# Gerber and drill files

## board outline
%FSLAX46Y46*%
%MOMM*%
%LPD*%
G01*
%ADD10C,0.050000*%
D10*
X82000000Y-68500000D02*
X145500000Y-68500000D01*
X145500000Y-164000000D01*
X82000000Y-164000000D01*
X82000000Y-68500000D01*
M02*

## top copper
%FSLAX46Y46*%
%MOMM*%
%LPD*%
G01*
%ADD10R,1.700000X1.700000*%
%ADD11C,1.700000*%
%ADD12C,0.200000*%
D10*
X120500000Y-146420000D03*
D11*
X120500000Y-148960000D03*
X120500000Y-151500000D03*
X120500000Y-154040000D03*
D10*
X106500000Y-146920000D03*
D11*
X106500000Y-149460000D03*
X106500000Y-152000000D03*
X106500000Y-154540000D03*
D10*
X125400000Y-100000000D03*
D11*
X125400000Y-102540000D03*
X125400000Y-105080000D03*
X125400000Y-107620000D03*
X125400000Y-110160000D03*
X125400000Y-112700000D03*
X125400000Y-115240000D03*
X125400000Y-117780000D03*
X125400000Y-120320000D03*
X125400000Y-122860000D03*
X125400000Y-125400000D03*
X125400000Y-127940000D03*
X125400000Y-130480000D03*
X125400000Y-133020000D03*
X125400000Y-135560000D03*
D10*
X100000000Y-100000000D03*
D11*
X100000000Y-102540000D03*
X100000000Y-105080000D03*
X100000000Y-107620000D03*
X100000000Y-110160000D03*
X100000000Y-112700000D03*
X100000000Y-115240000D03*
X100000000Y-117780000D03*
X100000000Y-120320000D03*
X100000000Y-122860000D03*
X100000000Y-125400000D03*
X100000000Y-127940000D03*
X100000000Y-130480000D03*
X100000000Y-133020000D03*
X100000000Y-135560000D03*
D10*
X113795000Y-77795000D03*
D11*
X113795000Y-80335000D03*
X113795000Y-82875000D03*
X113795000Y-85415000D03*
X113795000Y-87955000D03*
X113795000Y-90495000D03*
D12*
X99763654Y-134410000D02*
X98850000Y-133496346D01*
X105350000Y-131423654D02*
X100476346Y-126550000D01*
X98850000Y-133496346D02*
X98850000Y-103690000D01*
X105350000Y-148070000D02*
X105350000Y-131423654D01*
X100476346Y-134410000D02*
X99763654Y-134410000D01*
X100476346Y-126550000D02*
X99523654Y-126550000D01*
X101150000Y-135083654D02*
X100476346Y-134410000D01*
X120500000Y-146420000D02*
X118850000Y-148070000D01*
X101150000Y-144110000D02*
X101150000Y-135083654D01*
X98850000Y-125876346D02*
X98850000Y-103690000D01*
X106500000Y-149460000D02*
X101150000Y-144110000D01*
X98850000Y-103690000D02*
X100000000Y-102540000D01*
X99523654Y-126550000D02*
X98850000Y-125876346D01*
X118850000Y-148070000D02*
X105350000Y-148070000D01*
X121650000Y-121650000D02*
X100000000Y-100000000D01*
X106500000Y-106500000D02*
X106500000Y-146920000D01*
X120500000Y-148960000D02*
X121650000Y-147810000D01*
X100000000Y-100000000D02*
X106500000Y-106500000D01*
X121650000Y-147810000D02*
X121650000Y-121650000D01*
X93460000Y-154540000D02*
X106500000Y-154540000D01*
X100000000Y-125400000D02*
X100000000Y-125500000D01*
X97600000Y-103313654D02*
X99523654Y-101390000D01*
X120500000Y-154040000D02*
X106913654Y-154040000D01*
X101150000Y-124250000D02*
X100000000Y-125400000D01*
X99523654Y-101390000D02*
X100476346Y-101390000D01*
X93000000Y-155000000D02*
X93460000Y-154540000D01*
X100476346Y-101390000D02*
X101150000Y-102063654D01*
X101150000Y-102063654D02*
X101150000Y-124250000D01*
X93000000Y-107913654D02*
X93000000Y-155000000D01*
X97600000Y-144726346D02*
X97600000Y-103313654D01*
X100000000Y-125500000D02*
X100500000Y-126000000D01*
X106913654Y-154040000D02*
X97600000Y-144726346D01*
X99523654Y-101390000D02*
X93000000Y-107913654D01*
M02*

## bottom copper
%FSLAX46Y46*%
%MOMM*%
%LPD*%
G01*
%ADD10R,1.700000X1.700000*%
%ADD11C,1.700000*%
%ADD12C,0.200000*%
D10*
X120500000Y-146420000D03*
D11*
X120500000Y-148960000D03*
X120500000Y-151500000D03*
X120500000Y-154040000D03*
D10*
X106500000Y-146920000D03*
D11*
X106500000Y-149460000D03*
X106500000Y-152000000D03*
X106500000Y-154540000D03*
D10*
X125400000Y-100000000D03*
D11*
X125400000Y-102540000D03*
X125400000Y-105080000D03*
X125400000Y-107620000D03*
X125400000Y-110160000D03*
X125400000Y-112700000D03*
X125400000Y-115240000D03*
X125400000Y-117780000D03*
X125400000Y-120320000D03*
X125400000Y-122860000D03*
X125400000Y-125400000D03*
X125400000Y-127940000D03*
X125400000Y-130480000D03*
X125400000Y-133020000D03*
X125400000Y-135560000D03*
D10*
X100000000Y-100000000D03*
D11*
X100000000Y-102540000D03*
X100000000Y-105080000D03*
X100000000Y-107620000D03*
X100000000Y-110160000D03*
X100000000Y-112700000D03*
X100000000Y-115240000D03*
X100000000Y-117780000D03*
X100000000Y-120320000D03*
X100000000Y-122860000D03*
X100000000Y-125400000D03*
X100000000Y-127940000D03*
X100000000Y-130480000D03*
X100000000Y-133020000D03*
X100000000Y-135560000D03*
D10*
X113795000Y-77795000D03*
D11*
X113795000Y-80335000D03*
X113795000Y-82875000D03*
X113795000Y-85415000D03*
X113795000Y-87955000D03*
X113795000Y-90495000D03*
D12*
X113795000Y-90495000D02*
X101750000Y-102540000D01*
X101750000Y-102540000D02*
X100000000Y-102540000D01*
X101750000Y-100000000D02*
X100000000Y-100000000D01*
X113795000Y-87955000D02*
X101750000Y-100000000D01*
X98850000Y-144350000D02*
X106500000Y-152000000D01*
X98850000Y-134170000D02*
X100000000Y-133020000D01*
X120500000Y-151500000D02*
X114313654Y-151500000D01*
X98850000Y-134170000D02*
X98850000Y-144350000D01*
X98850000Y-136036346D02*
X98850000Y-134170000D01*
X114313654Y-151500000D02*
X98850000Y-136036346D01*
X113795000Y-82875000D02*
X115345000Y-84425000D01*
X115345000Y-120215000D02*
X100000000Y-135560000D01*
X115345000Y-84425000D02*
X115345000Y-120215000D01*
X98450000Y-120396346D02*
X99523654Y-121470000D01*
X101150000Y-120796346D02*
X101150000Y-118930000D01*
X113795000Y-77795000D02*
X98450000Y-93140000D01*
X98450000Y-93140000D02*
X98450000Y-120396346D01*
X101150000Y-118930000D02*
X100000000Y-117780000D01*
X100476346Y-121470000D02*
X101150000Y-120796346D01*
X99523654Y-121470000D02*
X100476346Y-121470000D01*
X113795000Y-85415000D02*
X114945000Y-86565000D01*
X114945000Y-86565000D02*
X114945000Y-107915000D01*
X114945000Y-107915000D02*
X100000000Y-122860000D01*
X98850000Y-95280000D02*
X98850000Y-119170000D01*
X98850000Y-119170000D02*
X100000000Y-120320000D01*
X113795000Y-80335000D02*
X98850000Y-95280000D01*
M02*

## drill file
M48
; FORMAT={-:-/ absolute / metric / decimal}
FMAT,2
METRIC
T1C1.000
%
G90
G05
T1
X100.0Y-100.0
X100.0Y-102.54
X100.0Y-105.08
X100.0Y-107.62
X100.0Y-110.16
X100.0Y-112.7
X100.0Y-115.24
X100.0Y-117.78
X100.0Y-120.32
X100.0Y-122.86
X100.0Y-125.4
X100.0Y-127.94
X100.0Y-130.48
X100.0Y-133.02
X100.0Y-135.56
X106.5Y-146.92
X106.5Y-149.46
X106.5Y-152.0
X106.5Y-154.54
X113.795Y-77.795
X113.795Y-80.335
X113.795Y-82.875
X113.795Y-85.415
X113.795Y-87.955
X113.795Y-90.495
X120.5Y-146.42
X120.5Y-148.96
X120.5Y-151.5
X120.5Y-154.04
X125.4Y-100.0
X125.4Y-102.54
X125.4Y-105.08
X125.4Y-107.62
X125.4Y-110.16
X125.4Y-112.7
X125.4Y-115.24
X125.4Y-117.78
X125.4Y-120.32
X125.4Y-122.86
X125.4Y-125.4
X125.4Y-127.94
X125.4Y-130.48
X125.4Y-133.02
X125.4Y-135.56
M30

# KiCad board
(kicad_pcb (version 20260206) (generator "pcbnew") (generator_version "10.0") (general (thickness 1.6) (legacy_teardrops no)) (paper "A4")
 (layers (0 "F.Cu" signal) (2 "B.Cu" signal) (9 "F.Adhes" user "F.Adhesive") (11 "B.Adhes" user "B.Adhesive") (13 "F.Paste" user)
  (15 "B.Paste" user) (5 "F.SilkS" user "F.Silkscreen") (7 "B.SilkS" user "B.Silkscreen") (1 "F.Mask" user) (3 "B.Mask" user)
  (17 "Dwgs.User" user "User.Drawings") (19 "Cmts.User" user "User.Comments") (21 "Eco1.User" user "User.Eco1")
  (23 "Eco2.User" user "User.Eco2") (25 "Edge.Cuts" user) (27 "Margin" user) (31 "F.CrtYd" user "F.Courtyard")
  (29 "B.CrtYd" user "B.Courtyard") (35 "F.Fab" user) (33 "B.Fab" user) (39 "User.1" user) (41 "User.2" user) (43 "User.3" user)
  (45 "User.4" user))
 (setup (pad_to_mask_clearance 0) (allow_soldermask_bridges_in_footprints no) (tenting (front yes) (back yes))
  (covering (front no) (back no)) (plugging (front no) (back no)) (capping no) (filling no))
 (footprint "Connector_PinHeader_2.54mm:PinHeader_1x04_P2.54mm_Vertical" (layer "F.Cu") (at 120.5 146.42)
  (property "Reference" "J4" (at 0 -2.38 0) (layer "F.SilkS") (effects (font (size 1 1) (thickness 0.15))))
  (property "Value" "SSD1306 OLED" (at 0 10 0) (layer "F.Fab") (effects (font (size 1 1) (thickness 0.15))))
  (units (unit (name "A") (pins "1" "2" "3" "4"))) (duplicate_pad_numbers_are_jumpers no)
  (pad "1" thru_hole rect (at 0 0) (size 1.7 1.7) (drill 1) (layers "*.Cu" "*.Mask") (remove_unused_layers no) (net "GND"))
  (pad "2" thru_hole circle (at 0 2.54) (size 1.7 1.7) (drill 1) (layers "*.Cu" "*.Mask") (remove_unused_layers no) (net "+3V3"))
  (pad "3" thru_hole circle (at 0 5.08) (size 1.7 1.7) (drill 1) (layers "*.Cu" "*.Mask") (remove_unused_layers no) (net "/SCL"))
  (pad "4" thru_hole circle (at 0 7.62) (size 1.7 1.7) (drill 1) (layers "*.Cu" "*.Mask") (remove_unused_layers no) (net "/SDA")))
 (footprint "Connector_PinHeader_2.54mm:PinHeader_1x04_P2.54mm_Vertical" (layer "F.Cu") (at 106.5 146.92)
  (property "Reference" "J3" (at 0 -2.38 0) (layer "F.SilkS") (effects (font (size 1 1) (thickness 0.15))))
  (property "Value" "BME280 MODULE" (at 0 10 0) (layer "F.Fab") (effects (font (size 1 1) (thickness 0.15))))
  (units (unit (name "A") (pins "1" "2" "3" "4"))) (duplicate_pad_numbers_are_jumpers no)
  (pad "1" thru_hole rect (at 0 0) (size 1.7 1.7) (drill 1) (layers "*.Cu" "*.Mask") (remove_unused_layers no) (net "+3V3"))
  (pad "2" thru_hole circle (at 0 2.54) (size 1.7 1.7) (drill 1) (layers "*.Cu" "*.Mask") (remove_unused_layers no) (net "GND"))
  (pad "3" thru_hole circle (at 0 5.08) (size 1.7 1.7) (drill 1) (layers "*.Cu" "*.Mask") (remove_unused_layers no) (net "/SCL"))
  (pad "4" thru_hole circle (at 0 7.62) (size 1.7 1.7) (drill 1) (layers "*.Cu" "*.Mask") (remove_unused_layers no) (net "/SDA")))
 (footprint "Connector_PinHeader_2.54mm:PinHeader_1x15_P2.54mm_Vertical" (layer "F.Cu") (at 125.4 100)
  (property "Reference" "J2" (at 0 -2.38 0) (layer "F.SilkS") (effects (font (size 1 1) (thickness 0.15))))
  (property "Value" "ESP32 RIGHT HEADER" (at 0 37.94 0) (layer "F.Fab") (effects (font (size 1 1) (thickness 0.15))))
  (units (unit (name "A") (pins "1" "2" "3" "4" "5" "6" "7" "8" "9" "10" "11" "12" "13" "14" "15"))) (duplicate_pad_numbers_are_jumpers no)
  (pad "1" thru_hole rect (at 0 0) (size 1.7 1.7) (drill 1) (layers "*.Cu" "*.Mask") (remove_unused_layers no)
   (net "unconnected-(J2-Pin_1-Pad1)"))
  (pad "2" thru_hole circle (at 0 2.54) (size 1.7 1.7) (drill 1) (layers "*.Cu" "*.Mask") (remove_unused_layers no)
   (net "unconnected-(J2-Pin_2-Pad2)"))
  (pad "3" thru_hole circle (at 0 5.08) (size 1.7 1.7) (drill 1) (layers "*.Cu" "*.Mask") (remove_unused_layers no)
   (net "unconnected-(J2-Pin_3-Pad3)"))
  (pad "4" thru_hole circle (at 0 7.62) (size 1.7 1.7) (drill 1) (layers "*.Cu" "*.Mask") (remove_unused_layers no)
   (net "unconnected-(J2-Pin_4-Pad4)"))
  (pad "5" thru_hole circle (at 0 10.16) (size 1.7 1.7) (drill 1) (layers "*.Cu" "*.Mask") (remove_unused_layers no)
   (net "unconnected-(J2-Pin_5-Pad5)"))
  (pad "6" thru_hole circle (at 0 12.7) (size 1.7 1.7) (drill 1) (layers "*.Cu" "*.Mask") (remove_unused_layers no)
   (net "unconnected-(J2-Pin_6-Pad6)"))
  (pad "7" thru_hole circle (at 0 15.24) (size 1.7 1.7) (drill 1) (layers "*.Cu" "*.Mask") (remove_unused_layers no)
   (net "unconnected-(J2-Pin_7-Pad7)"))
  (pad "8" thru_hole circle (at 0 17.78) (size 1.7 1.7) (drill 1) (layers "*.Cu" "*.Mask") (remove_unused_layers no)
   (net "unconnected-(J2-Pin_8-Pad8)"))
  (pad "9" thru_hole circle (at 0 20.32) (size 1.7 1.7) (drill 1) (layers "*.Cu" "*.Mask") (remove_unused_layers no)
   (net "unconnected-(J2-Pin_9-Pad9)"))
  (pad "10" thru_hole circle (at 0 22.86) (size 1.7 1.7) (drill 1) (layers "*.Cu" "*.Mask") (remove_unused_layers no)
   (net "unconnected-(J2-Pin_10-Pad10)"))
  (pad "11" thru_hole circle (at 0 25.4) (size 1.7 1.7) (drill 1) (layers "*.Cu" "*.Mask") (remove_unused_layers no)
   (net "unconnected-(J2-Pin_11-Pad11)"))
  (pad "12" thru_hole circle (at 0 27.94) (size 1.7 1.7) (drill 1) (layers "*.Cu" "*.Mask") (remove_unused_layers no)
   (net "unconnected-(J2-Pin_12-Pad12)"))
  (pad "13" thru_hole circle (at 0 30.48) (size 1.7 1.7) (drill 1) (layers "*.Cu" "*.Mask") (remove_unused_layers no)
   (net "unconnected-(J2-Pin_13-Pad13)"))
  (pad "14" thru_hole circle (at 0 33.02) (size 1.7 1.7) (drill 1) (layers "*.Cu" "*.Mask") (remove_unused_layers no)
   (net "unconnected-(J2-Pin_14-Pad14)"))
  (pad "15" thru_hole circle (at 0 35.56) (size 1.7 1.7) (drill 1) (layers "*.Cu" "*.Mask") (remove_unused_layers no)
   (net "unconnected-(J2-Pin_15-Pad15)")))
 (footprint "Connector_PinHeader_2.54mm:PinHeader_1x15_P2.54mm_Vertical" (layer "F.Cu") (at 100 100)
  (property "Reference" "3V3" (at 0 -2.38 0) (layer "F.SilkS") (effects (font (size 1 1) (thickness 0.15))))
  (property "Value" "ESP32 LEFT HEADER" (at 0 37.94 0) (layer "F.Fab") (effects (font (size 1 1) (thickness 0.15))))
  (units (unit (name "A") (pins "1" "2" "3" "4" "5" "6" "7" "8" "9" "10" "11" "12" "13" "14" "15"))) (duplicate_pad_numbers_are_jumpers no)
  (pad "1" thru_hole rect (at 0 0) (size 1.7 1.7) (drill 1) (layers "*.Cu" "*.Mask") (remove_unused_layers no) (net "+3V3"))
  (pad "2" thru_hole circle (at 0 2.54) (size 1.7 1.7) (drill 1) (layers "*.Cu" "*.Mask") (remove_unused_layers no) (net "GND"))
  (pad "3" thru_hole circle (at 0 5.08) (size 1.7 1.7) (drill 1) (layers "*.Cu" "*.Mask") (remove_unused_layers no)
   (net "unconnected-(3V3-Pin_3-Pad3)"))
  (pad "4" thru_hole circle (at 0 7.62) (size 1.7 1.7) (drill 1) (layers "*.Cu" "*.Mask") (remove_unused_layers no)
   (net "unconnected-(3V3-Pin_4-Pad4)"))
  (pad "5" thru_hole circle (at 0 10.16) (size 1.7 1.7) (drill 1) (layers "*.Cu" "*.Mask") (remove_unused_layers no)
   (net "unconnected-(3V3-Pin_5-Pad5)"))
  (pad "6" thru_hole circle (at 0 12.7) (size 1.7 1.7) (drill 1) (layers "*.Cu" "*.Mask") (remove_unused_layers no)
   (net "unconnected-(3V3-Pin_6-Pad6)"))
  (pad "7" thru_hole circle (at 0 15.24) (size 1.7 1.7) (drill 1) (layers "*.Cu" "*.Mask") (remove_unused_layers no)
   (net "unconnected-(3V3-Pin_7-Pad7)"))
  (pad "8" thru_hole circle (at 0 17.78) (size 1.7 1.7) (drill 1) (layers "*.Cu" "*.Mask") (remove_unused_layers no) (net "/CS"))
  (pad "9" thru_hole circle (at 0 20.32) (size 1.7 1.7) (drill 1) (layers "*.Cu" "*.Mask") (remove_unused_layers no) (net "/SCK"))
  (pad "10" thru_hole circle (at 0 22.86) (size 1.7 1.7) (drill 1) (layers "*.Cu" "*.Mask") (remove_unused_layers no) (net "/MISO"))
  (pad "11" thru_hole circle (at 0 25.4) (size 1.7 1.7) (drill 1) (layers "*.Cu" "*.Mask") (remove_unused_layers no) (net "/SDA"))
  (pad "12" thru_hole circle (at 0 27.94) (size 1.7 1.7) (drill 1) (layers "*.Cu" "*.Mask") (remove_unused_layers no)
   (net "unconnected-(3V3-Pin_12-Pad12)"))
  (pad "13" thru_hole circle (at 0 30.48) (size 1.7 1.7) (drill 1) (layers "*.Cu" "*.Mask") (remove_unused_layers no)
   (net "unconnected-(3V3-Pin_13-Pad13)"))
  (pad "14" thru_hole circle (at 0 33.02) (size 1.7 1.7) (drill 1) (layers "*.Cu" "*.Mask") (remove_unused_layers no) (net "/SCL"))
  (pad "15" thru_hole circle (at 0 35.56) (size 1.7 1.7) (drill 1) (layers "*.Cu" "*.Mask") (remove_unused_layers no) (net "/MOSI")))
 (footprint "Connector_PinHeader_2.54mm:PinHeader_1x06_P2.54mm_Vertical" (layer "F.Cu") (at 113.795 77.795)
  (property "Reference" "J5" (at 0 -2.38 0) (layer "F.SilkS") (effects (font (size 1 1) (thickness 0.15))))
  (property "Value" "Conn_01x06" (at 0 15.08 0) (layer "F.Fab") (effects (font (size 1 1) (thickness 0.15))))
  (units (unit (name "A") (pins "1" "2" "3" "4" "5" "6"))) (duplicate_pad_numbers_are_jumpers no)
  (pad "1" thru_hole rect (at 0 0) (size 1.7 1.7) (drill 1) (layers "*.Cu" "*.Mask") (remove_unused_layers no) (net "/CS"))
  (pad "2" thru_hole circle (at 0 2.54) (size 1.7 1.7) (drill 1) (layers "*.Cu" "*.Mask") (remove_unused_layers no) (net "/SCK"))
  (pad "3" thru_hole circle (at 0 5.08) (size 1.7 1.7) (drill 1) (layers "*.Cu" "*.Mask") (remove_unused_layers no) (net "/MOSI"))
  (pad "4" thru_hole circle (at 0 7.62) (size 1.7 1.7) (drill 1) (layers "*.Cu" "*.Mask") (remove_unused_layers no) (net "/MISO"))
  (pad "5" thru_hole circle (at 0 10.16) (size 1.7 1.7) (drill 1) (layers "*.Cu" "*.Mask") (remove_unused_layers no) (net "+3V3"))
  (pad "6" thru_hole circle (at 0 12.7) (size 1.7 1.7) (drill 1) (layers "*.Cu" "*.Mask") (remove_unused_layers no) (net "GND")))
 (gr_rect (start 82 68.5) (end 145.5 164) (stroke (width 0.05) (type default)) (fill no) (layer "Edge.Cuts"))
 (segment (start 99.763654 134.41) (end 98.85 133.496346) (width 0.2) (layer "F.Cu") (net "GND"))
 (segment (start 105.35 131.423654) (end 100.476346 126.55) (width 0.2) (layer "F.Cu") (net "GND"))
 (segment (start 98.85 133.496346) (end 98.85 103.69) (width 0.2) (layer "F.Cu") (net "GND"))
 (segment (start 105.35 148.07) (end 105.35 131.423654) (width 0.2) (layer "F.Cu") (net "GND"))
 (segment (start 100.476346 134.41) (end 99.763654 134.41) (width 0.2) (layer "F.Cu") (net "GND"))
 (segment (start 100.476346 126.55) (end 99.523654 126.55) (width 0.2) (layer "F.Cu") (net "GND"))
 (segment (start 101.15 135.083654) (end 100.476346 134.41) (width 0.2) (layer "F.Cu") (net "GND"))
 (segment (start 120.5 146.42) (end 118.85 148.07) (width 0.2) (layer "F.Cu") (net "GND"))
 (segment (start 101.15 144.11) (end 101.15 135.083654) (width 0.2) (layer "F.Cu") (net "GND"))
 (segment (start 98.85 125.876346) (end 98.85 103.69) (width 0.2) (layer "F.Cu") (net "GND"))
 (segment (start 106.5 149.46) (end 101.15 144.11) (width 0.2) (layer "F.Cu") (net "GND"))
 (segment (start 98.85 103.69) (end 100 102.54) (width 0.2) (layer "F.Cu") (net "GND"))
 (segment (start 99.523654 126.55) (end 98.85 125.876346) (width 0.2) (layer "F.Cu") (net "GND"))
 (segment (start 118.85 148.07) (end 105.35 148.07) (width 0.2) (layer "F.Cu") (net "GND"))
 (segment (start 113.795 90.495) (end 101.75 102.54) (width 0.2) (layer "B.Cu") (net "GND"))
 (segment (start 101.75 102.54) (end 100 102.54) (width 0.2) (layer "B.Cu") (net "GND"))
 (segment (start 121.65 121.65) (end 100 100) (width 0.2) (layer "F.Cu") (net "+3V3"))
 (segment (start 106.5 106.5) (end 106.5 146.92) (width 0.2) (layer "F.Cu") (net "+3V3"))
 (segment (start 120.5 148.96) (end 121.65 147.81) (width 0.2) (layer "F.Cu") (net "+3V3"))
 (segment (start 100 100) (end 106.5 106.5) (width 0.2) (layer "F.Cu") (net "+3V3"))
 (segment (start 121.65 147.81) (end 121.65 121.65) (width 0.2) (layer "F.Cu") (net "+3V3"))
 (segment (start 101.75 100) (end 100 100) (width 0.2) (layer "B.Cu") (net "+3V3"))
 (segment (start 113.795 87.955) (end 101.75 100) (width 0.2) (layer "B.Cu") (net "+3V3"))
 (segment (start 98.85 144.35) (end 106.5 152) (width 0.2) (layer "B.Cu") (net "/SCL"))
 (segment (start 98.85 134.17) (end 100 133.02) (width 0.2) (layer "B.Cu") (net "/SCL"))
 (segment (start 120.5 151.5) (end 114.313654 151.5) (width 0.2) (layer "B.Cu") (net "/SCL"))
 (segment (start 98.85 134.17) (end 98.85 144.35) (width 0.2) (layer "B.Cu") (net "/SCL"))
 (segment (start 98.85 136.036346) (end 98.85 134.17) (width 0.2) (layer "B.Cu") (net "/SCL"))
 (segment (start 114.313654 151.5) (end 98.85 136.036346) (width 0.2) (layer "B.Cu") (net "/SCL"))
 (segment (start 93.46 154.54) (end 106.5 154.54) (width 0.2) (layer "F.Cu") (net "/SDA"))
 (segment (start 100 125.4) (end 100 125.5) (width 0.2) (layer "F.Cu") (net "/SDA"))
 (segment (start 97.6 103.313654) (end 99.523654 101.39) (width 0.2) (layer "F.Cu") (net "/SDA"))
 (segment (start 120.5 154.04) (end 106.913654 154.04) (width 0.2) (layer "F.Cu") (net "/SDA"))
 (segment (start 101.15 124.25) (end 100 125.4) (width 0.2) (layer "F.Cu") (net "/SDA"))
 (segment (start 99.523654 101.39) (end 100.476346 101.39) (width 0.2) (layer "F.Cu") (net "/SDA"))
 (segment (start 93 155) (end 93.46 154.54) (width 0.2) (layer "F.Cu") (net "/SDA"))
 (segment (start 100.476346 101.39) (end 101.15 102.063654) (width 0.2) (layer "F.Cu") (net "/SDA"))
 (segment (start 101.15 102.063654) (end 101.15 124.25) (width 0.2) (layer "F.Cu") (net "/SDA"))
 (segment (start 93 107.913654) (end 93 155) (width 0.2) (layer "F.Cu") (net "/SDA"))
 (segment (start 97.6 144.726346) (end 97.6 103.313654) (width 0.2) (layer "F.Cu") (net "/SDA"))
 (segment (start 100 125.5) (end 100.5 126) (width 0.2) (layer "F.Cu") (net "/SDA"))
 (segment (start 106.913654 154.04) (end 97.6 144.726346) (width 0.2) (layer "F.Cu") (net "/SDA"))
 (segment (start 99.523654 101.39) (end 93 107.913654) (width 0.2) (layer "F.Cu") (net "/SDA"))
 (segment (start 113.795 82.875) (end 115.345 84.425) (width 0.2) (layer "B.Cu") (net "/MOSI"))
 (segment (start 115.345 120.215) (end 100 135.56) (width 0.2) (layer "B.Cu") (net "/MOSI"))
 (segment (start 115.345 84.425) (end 115.345 120.215) (width 0.2) (layer "B.Cu") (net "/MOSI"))
 (segment (start 98.45 120.396346) (end 99.523654 121.47) (width 0.2) (layer "B.Cu") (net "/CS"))
 (segment (start 101.15 120.796346) (end 101.15 118.93) (width 0.2) (layer "B.Cu") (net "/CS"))
 (segment (start 113.795 77.795) (end 98.45 93.14) (width 0.2) (layer "B.Cu") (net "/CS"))
 (segment (start 98.45 93.14) (end 98.45 120.396346) (width 0.2) (layer "B.Cu") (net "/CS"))
 (segment (start 101.15 118.93) (end 100 117.78) (width 0.2) (layer "B.Cu") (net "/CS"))
 (segment (start 100.476346 121.47) (end 101.15 120.796346) (width 0.2) (layer "B.Cu") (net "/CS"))
 (segment (start 99.523654 121.47) (end 100.476346 121.47) (width 0.2) (layer "B.Cu") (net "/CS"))
 (segment (start 113.795 85.415) (end 114.945 86.565) (width 0.2) (layer "B.Cu") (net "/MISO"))
 (segment (start 114.945 86.565) (end 114.945 107.915) (width 0.2) (layer "B.Cu") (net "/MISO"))
 (segment (start 114.945 107.915) (end 100 122.86) (width 0.2) (layer "B.Cu") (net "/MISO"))
 (segment (start 98.85 95.28) (end 98.85 119.17) (width 0.2) (layer "B.Cu") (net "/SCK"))
 (segment (start 98.85 119.17) (end 100 120.32) (width 0.2) (layer "B.Cu") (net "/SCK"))
 (segment (start 113.795 80.335) (end 98.85 95.28) (width 0.2) (layer "B.Cu") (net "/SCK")))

